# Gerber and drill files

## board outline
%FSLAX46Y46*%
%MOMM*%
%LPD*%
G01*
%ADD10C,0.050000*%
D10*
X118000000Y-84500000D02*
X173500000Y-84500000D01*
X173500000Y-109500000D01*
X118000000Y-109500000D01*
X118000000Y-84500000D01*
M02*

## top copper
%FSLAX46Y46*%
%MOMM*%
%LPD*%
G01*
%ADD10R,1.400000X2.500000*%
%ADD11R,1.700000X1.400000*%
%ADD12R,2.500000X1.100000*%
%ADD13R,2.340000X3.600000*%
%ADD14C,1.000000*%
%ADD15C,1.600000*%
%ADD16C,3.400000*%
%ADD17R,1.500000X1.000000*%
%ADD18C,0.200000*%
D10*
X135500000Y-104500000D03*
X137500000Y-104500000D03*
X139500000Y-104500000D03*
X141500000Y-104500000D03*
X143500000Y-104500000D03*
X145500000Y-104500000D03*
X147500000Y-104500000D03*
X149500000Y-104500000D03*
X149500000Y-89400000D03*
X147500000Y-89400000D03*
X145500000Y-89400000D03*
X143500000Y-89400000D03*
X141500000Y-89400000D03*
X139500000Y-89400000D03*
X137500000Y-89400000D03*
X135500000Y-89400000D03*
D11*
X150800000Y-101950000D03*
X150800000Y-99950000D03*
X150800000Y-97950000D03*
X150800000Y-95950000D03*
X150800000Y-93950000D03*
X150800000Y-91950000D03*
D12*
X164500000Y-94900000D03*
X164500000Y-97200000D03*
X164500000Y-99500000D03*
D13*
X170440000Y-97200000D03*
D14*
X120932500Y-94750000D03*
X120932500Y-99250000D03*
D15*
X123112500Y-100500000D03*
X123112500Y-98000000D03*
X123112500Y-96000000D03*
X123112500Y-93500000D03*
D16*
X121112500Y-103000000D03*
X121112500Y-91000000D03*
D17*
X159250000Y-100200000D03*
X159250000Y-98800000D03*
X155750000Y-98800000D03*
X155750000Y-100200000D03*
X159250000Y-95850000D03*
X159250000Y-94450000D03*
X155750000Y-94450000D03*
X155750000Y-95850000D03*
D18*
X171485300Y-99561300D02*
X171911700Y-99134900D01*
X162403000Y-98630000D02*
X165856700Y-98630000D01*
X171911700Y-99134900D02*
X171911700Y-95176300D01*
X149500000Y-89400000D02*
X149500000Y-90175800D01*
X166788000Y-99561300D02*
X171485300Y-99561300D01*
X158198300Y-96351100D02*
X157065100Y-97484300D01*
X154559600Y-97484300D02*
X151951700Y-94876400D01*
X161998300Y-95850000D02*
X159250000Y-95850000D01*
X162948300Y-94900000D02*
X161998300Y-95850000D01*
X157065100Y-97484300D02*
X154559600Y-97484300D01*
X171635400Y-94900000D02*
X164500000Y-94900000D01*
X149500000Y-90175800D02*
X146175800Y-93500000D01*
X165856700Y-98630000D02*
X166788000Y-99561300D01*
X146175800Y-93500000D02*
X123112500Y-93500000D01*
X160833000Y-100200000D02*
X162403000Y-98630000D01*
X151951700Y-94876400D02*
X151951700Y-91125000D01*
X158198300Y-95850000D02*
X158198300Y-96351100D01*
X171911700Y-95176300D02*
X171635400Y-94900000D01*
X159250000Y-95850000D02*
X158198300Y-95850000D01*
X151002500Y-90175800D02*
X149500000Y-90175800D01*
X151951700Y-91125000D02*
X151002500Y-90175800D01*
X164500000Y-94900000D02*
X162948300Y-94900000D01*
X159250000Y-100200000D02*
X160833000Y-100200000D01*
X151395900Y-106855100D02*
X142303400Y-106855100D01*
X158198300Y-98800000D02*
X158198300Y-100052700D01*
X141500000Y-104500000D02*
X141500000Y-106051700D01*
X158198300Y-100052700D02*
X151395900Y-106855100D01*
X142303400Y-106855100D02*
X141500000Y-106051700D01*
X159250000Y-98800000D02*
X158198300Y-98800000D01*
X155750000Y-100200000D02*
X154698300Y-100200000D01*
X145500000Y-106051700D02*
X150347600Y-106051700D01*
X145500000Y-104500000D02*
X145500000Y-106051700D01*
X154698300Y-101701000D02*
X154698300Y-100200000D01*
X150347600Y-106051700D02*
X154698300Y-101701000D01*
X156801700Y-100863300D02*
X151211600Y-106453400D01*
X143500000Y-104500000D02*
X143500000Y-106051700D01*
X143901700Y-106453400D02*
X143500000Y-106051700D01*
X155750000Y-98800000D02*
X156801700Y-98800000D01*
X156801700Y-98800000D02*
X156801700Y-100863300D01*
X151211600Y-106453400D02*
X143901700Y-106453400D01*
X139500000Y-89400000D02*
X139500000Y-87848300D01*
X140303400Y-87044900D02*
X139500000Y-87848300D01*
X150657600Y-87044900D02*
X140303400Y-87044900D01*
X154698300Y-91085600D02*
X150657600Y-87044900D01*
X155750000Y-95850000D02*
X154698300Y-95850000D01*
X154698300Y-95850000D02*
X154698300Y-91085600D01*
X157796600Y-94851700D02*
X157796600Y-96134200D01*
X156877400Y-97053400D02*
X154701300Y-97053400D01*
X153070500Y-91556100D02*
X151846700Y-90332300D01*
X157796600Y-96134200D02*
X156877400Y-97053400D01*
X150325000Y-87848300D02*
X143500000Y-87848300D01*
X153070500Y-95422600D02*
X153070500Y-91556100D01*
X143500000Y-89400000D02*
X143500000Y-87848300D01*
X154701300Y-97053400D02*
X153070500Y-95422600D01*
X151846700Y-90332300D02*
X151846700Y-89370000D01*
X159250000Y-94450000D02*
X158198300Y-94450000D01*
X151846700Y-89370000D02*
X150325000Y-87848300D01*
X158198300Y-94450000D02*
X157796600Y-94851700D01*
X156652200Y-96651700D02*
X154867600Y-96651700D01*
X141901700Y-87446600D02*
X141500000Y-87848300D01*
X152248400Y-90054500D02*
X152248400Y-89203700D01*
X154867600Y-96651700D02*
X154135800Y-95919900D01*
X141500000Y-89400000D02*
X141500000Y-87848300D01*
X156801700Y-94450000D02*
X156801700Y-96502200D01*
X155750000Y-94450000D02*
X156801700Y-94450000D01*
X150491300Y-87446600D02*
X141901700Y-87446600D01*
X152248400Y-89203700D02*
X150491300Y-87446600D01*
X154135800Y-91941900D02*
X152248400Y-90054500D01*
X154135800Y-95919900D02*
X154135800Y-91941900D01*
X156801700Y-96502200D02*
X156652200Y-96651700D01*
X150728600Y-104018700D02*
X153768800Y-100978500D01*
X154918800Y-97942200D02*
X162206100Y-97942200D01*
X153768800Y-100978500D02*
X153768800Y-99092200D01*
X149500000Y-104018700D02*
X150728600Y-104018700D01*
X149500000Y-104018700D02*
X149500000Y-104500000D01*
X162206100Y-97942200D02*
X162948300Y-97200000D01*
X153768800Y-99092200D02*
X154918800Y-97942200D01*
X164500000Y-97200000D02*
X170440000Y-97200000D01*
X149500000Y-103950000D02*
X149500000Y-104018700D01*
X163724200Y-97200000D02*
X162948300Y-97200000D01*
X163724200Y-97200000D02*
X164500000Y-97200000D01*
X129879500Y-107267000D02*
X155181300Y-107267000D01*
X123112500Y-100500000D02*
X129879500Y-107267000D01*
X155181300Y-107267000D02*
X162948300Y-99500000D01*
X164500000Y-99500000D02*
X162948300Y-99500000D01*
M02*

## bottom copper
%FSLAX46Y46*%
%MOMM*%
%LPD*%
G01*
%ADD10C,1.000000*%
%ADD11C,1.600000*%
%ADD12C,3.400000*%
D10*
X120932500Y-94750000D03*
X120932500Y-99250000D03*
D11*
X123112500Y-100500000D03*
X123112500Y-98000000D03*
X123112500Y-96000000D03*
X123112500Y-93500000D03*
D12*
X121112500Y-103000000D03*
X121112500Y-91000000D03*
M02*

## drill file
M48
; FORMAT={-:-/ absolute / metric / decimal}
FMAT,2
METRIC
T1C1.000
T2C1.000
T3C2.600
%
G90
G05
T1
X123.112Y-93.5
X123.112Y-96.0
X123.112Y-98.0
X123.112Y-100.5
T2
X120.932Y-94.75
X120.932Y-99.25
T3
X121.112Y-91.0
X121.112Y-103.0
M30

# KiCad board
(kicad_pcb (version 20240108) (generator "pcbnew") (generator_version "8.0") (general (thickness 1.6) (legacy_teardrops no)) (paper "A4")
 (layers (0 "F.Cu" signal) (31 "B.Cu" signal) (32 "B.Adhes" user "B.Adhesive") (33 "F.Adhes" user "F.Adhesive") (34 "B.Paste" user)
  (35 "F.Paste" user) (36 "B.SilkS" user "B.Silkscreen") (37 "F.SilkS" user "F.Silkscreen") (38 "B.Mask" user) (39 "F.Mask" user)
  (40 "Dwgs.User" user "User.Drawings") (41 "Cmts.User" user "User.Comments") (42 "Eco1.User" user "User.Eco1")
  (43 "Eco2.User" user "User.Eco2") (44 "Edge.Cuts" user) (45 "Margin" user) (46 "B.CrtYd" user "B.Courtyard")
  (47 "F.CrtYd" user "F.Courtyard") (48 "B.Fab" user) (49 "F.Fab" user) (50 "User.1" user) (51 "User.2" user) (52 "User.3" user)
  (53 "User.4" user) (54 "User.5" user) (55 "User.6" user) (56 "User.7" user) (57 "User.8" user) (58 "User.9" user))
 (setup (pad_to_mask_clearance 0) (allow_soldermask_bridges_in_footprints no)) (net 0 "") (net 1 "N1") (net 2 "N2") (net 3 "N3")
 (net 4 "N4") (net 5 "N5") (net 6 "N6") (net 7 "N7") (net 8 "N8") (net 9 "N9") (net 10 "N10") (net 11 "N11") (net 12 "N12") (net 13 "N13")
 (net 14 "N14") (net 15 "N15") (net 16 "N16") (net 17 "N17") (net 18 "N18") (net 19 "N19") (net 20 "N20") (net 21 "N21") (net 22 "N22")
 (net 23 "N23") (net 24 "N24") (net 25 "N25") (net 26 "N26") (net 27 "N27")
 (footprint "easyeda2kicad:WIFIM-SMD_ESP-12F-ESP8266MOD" (layer "F.Cu") (at 143.15 96.95)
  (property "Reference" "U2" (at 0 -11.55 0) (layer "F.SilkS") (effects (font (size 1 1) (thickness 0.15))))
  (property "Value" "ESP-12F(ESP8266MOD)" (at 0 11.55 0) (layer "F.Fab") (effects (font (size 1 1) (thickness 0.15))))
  (pad "1" smd rect (at -7.65 7.55 90) (size 2.5 1.4) (layers "F.Cu" "F.Paste" "F.Mask") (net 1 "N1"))
  (pad "2" smd rect (at -5.65 7.55 90) (size 2.5 1.4) (layers "F.Cu" "F.Paste" "F.Mask") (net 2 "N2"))
  (pad "3" smd rect (at -3.65 7.55 90) (size 2.5 1.4) (layers "F.Cu" "F.Paste" "F.Mask") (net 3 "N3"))
  (pad "4" smd rect (at -1.65 7.55 90) (size 2.5 1.4) (layers "F.Cu" "F.Paste" "F.Mask") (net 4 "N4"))
  (pad "5" smd rect (at 0.35 7.55 90) (size 2.5 1.4) (layers "F.Cu" "F.Paste" "F.Mask") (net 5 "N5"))
  (pad "6" smd rect (at 2.35 7.55 90) (size 2.5 1.4) (layers "F.Cu" "F.Paste" "F.Mask") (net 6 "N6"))
  (pad "7" smd rect (at 4.35 7.55 90) (size 2.5 1.4) (layers "F.Cu" "F.Paste" "F.Mask") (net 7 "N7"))
  (pad "8" smd rect (at 6.35 7.55 90) (size 2.5 1.4) (layers "F.Cu" "F.Paste" "F.Mask") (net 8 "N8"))
  (pad "9" smd rect (at 6.35 -7.55 270) (size 2.5 1.4) (layers "F.Cu" "F.Paste" "F.Mask") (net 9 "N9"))
  (pad "10" smd rect (at 4.35 -7.55 270) (size 2.5 1.4) (layers "F.Cu" "F.Paste" "F.Mask") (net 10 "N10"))
  (pad "11" smd rect (at 2.35 -7.55 270) (size 2.5 1.4) (layers "F.Cu" "F.Paste" "F.Mask") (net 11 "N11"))
  (pad "12" smd rect (at 0.35 -7.55 270) (size 2.5 1.4) (layers "F.Cu" "F.Paste" "F.Mask") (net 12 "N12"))
  (pad "13" smd rect (at -1.65 -7.55 270) (size 2.5 1.4) (layers "F.Cu" "F.Paste" "F.Mask") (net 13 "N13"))
  (pad "14" smd rect (at -3.65 -7.55 270) (size 2.5 1.4) (layers "F.Cu" "F.Paste" "F.Mask") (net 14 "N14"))
  (pad "15" smd rect (at -5.65 -7.55 270) (size 2.5 1.4) (layers "F.Cu" "F.Paste" "F.Mask") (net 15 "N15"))
  (pad "16" smd rect (at -7.65 -7.55 270) (size 2.5 1.4) (layers "F.Cu" "F.Paste" "F.Mask") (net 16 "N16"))
  (pad "17" smd rect (at 7.65 5 180) (size 1.7 1.4) (layers "F.Cu" "F.Paste" "F.Mask") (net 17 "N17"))
  (pad "18" smd rect (at 7.65 3 180) (size 1.7 1.4) (layers "F.Cu" "F.Paste" "F.Mask") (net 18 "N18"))
  (pad "19" smd rect (at 7.65 1 180) (size 1.7 1.4) (layers "F.Cu" "F.Paste" "F.Mask") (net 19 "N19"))
  (pad "20" smd rect (at 7.65 -1 180) (size 1.7 1.4) (layers "F.Cu" "F.Paste" "F.Mask") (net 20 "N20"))
  (pad "21" smd rect (at 7.65 -3 180) (size 1.7 1.4) (layers "F.Cu" "F.Paste" "F.Mask") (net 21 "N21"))
  (pad "22" smd rect (at 7.65 -5 180) (size 1.7 1.4) (layers "F.Cu" "F.Paste" "F.Mask") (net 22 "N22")))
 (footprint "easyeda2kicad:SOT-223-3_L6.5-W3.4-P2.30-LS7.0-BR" (layer "F.Cu") (at 167.47 97.2 180)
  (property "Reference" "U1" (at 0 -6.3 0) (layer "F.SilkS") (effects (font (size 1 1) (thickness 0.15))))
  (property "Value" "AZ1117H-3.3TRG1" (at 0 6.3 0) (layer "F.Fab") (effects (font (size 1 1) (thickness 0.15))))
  (pad "1" smd rect (at 2.97 2.3 180) (size 2.5 1.1) (layers "F.Cu" "F.Paste" "F.Mask") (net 9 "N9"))
  (pad "2" smd rect (at 2.97 0 180) (size 2.5 1.1) (layers "F.Cu" "F.Paste" "F.Mask") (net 8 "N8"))
  (pad "3" smd rect (at 2.97 -2.3 180) (size 2.5 1.1) (layers "F.Cu" "F.Paste" "F.Mask") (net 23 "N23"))
  (pad "4" smd rect (at -2.97 0 180) (size 2.34 3.6) (layers "F.Cu" "F.Paste" "F.Mask") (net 8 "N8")))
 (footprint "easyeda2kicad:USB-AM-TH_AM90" (layer "F.Cu") (at 122.1125 97 -90)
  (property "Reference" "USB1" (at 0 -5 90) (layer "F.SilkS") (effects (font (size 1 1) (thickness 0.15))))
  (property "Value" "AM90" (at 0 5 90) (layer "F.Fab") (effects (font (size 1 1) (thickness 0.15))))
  (pad "" thru_hole circle (at -2.25 1.18 270) (size 1 1) (drill 1) (layers "*.Cu" "*.Mask") (remove_unused_layers no))
  (pad "" thru_hole circle (at 2.25 1.18 270) (size 1 1) (drill 1) (layers "*.Cu" "*.Mask") (remove_unused_layers no))
  (pad "1" thru_hole circle (at 3.5 -1 180) (size 1.6 1.6) (drill 0.999998) (layers "*.Cu" "*.Mask") (remove_unused_layers no)
   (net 23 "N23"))
  (pad "2" thru_hole circle (at 1 -1 180) (size 1.6 1.6) (drill 0.999998) (layers "*.Cu" "*.Mask") (remove_unused_layers no) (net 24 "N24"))
  (pad "3" thru_hole circle (at -1 -1 180) (size 1.6 1.6) (drill 0.999998) (layers "*.Cu" "*.Mask") (remove_unused_layers no) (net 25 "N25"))
  (pad "4" thru_hole circle (at -3.5 -1 180) (size 1.6 1.6) (drill 0.999998) (layers "*.Cu" "*.Mask") (remove_unused_layers no) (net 9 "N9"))
  (pad "MH1" thru_hole circle (at 6 1 180) (size 3.4 3.4) (drill 2.599995) (layers "*.Cu" "*.Mask") (remove_unused_layers no) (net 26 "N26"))
  (pad "MH2" thru_hole circle (at -6 1 180) (size 3.4 3.4) (drill 2.599995) (layers "*.Cu" "*.Mask") (remove_unused_layers no)
   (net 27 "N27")))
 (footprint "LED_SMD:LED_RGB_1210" (layer "F.Cu") (at 157.5 99.5 180)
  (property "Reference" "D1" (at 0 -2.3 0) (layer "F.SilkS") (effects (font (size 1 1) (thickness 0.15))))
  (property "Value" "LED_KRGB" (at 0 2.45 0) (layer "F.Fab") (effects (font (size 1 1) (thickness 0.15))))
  (pad "1" smd rect (at -1.75 -0.7) (size 1.5 1) (layers "F.Cu" "F.Paste" "F.Mask") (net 9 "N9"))
  (pad "2" smd rect (at -1.75 0.7) (size 1.5 1) (layers "F.Cu" "F.Paste" "F.Mask") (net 4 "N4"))
  (pad "3" smd rect (at 1.75 0.7) (size 1.5 1) (layers "F.Cu" "F.Paste" "F.Mask") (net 5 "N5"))
  (pad "4" smd rect (at 1.75 -0.7) (size 1.5 1) (layers "F.Cu" "F.Paste" "F.Mask") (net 6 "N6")))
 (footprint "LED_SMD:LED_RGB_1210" (layer "F.Cu") (at 157.5 95.15 180)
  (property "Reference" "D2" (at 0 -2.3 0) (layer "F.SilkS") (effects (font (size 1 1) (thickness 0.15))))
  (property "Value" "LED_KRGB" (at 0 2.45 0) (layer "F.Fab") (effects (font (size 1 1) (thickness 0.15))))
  (pad "1" smd rect (at -1.75 -0.7) (size 1.5 1) (layers "F.Cu" "F.Paste" "F.Mask") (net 9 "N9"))
  (pad "2" smd rect (at -1.75 0.7) (size 1.5 1) (layers "F.Cu" "F.Paste" "F.Mask") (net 12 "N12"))
  (pad "3" smd rect (at 1.75 0.7) (size 1.5 1) (layers "F.Cu" "F.Paste" "F.Mask") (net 13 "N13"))
  (pad "4" smd rect (at 1.75 -0.7) (size 1.5 1) (layers "F.Cu" "F.Paste" "F.Mask") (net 14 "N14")))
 (gr_rect (start 118 84.5) (end 173.5 109.5) (stroke (width 0.05) (type default)) (fill none) (layer "Edge.Cuts"))
 (segment (start 171.4853 99.5613) (end 171.9117 99.1349) (width 0.2) (layer "F.Cu") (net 9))
 (segment (start 162.403 98.63) (end 165.8567 98.63) (width 0.2) (layer "F.Cu") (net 9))
 (segment (start 171.9117 99.1349) (end 171.9117 95.1763) (width 0.2) (layer "F.Cu") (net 9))
 (segment (start 149.5 89.4) (end 149.5 90.1758) (width 0.2) (layer "F.Cu") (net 9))
 (segment (start 166.788 99.5613) (end 171.4853 99.5613) (width 0.2) (layer "F.Cu") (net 9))
 (segment (start 158.1983 96.3511) (end 157.0651 97.4843) (width 0.2) (layer "F.Cu") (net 9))
 (segment (start 154.5596 97.4843) (end 151.9517 94.8764) (width 0.2) (layer "F.Cu") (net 9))
 (segment (start 161.9983 95.85) (end 159.25 95.85) (width 0.2) (layer "F.Cu") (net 9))
 (segment (start 162.9483 94.9) (end 161.9983 95.85) (width 0.2) (layer "F.Cu") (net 9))
 (segment (start 157.0651 97.4843) (end 154.5596 97.4843) (width 0.2) (layer "F.Cu") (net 9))
 (segment (start 171.6354 94.9) (end 164.5 94.9) (width 0.2) (layer "F.Cu") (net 9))
 (segment (start 149.5 90.1758) (end 146.1758 93.5) (width 0.2) (layer "F.Cu") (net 9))
 (segment (start 165.8567 98.63) (end 166.788 99.5613) (width 0.2) (layer "F.Cu") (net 9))
 (segment (start 146.1758 93.5) (end 123.1125 93.5) (width 0.2) (layer "F.Cu") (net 9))
 (segment (start 160.833 100.2) (end 162.403 98.63) (width 0.2) (layer "F.Cu") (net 9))
 (segment (start 151.9517 94.8764) (end 151.9517 91.125) (width 0.2) (layer "F.Cu") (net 9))
 (segment (start 158.1983 95.85) (end 158.1983 96.3511) (width 0.2) (layer "F.Cu") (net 9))
 (segment (start 171.9117 95.1763) (end 171.6354 94.9) (width 0.2) (layer "F.Cu") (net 9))
 (segment (start 159.25 95.85) (end 158.1983 95.85) (width 0.2) (layer "F.Cu") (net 9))
 (segment (start 151.0025 90.1758) (end 149.5 90.1758) (width 0.2) (layer "F.Cu") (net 9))
 (segment (start 151.9517 91.125) (end 151.0025 90.1758) (width 0.2) (layer "F.Cu") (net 9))
 (segment (start 164.5 94.9) (end 162.9483 94.9) (width 0.2) (layer "F.Cu") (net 9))
 (segment (start 159.25 100.2) (end 160.833 100.2) (width 0.2) (layer "F.Cu") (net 9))
 (segment (start 151.3959 106.8551) (end 142.3034 106.8551) (width 0.2) (layer "F.Cu") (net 4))
 (segment (start 158.1983 98.8) (end 158.1983 100.0527) (width 0.2) (layer "F.Cu") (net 4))
 (segment (start 141.5 104.5) (end 141.5 106.0517) (width 0.2) (layer "F.Cu") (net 4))
 (segment (start 158.1983 100.0527) (end 151.3959 106.8551) (width 0.2) (layer "F.Cu") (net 4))
 (segment (start 142.3034 106.8551) (end 141.5 106.0517) (width 0.2) (layer "F.Cu") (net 4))
 (segment (start 159.25 98.8) (end 158.1983 98.8) (width 0.2) (layer "F.Cu") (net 4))
 (segment (start 155.75 100.2) (end 154.6983 100.2) (width 0.2) (layer "F.Cu") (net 6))
 (segment (start 145.5 106.0517) (end 150.3476 106.0517) (width 0.2) (layer "F.Cu") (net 6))
 (segment (start 145.5 104.5) (end 145.5 106.0517) (width 0.2) (layer "F.Cu") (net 6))
 (segment (start 154.6983 101.701) (end 154.6983 100.2) (width 0.2) (layer "F.Cu") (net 6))
 (segment (start 150.3476 106.0517) (end 154.6983 101.701) (width 0.2) (layer "F.Cu") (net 6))
 (segment (start 156.8017 100.8633) (end 151.2116 106.4534) (width 0.2) (layer "F.Cu") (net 5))
 (segment (start 143.5 104.5) (end 143.5 106.0517) (width 0.2) (layer "F.Cu") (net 5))
 (segment (start 143.9017 106.4534) (end 143.5 106.0517) (width 0.2) (layer "F.Cu") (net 5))
 (segment (start 155.75 98.8) (end 156.8017 98.8) (width 0.2) (layer "F.Cu") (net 5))
 (segment (start 156.8017 98.8) (end 156.8017 100.8633) (width 0.2) (layer "F.Cu") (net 5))
 (segment (start 151.2116 106.4534) (end 143.9017 106.4534) (width 0.2) (layer "F.Cu") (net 5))
 (segment (start 139.5 89.4) (end 139.5 87.8483) (width 0.2) (layer "F.Cu") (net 14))
 (segment (start 140.3034 87.0449) (end 139.5 87.8483) (width 0.2) (layer "F.Cu") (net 14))
 (segment (start 150.6576 87.0449) (end 140.3034 87.0449) (width 0.2) (layer "F.Cu") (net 14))
 (segment (start 154.6983 91.0856) (end 150.6576 87.0449) (width 0.2) (layer "F.Cu") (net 14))
 (segment (start 155.75 95.85) (end 154.6983 95.85) (width 0.2) (layer "F.Cu") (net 14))
 (segment (start 154.6983 95.85) (end 154.6983 91.0856) (width 0.2) (layer "F.Cu") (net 14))
 (segment (start 157.7966 94.8517) (end 157.7966 96.1342) (width 0.2) (layer "F.Cu") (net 12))
 (segment (start 156.8774 97.0534) (end 154.7013 97.0534) (width 0.2) (layer "F.Cu") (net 12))
 (segment (start 153.0705 91.5561) (end 151.8467 90.3323) (width 0.2) (layer "F.Cu") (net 12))
 (segment (start 157.7966 96.1342) (end 156.8774 97.0534) (width 0.2) (layer "F.Cu") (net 12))
 (segment (start 150.325 87.8483) (end 143.5 87.8483) (width 0.2) (layer "F.Cu") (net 12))
 (segment (start 153.0705 95.4226) (end 153.0705 91.5561) (width 0.2) (layer "F.Cu") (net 12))
 (segment (start 143.5 89.4) (end 143.5 87.8483) (width 0.2) (layer "F.Cu") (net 12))
 (segment (start 154.7013 97.0534) (end 153.0705 95.4226) (width 0.2) (layer "F.Cu") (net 12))
 (segment (start 151.8467 90.3323) (end 151.8467 89.37) (width 0.2) (layer "F.Cu") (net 12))
 (segment (start 159.25 94.45) (end 158.1983 94.45) (width 0.2) (layer "F.Cu") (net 12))
 (segment (start 151.8467 89.37) (end 150.325 87.8483) (width 0.2) (layer "F.Cu") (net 12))
 (segment (start 158.1983 94.45) (end 157.7966 94.8517) (width 0.2) (layer "F.Cu") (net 12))
 (segment (start 156.6522 96.6517) (end 154.8676 96.6517) (width 0.2) (layer "F.Cu") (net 13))
 (segment (start 141.9017 87.4466) (end 141.5 87.8483) (width 0.2) (layer "F.Cu") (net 13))
 (segment (start 152.2484 90.0545) (end 152.2484 89.2037) (width 0.2) (layer "F.Cu") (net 13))
 (segment (start 154.8676 96.6517) (end 154.1358 95.9199) (width 0.2) (layer "F.Cu") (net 13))
 (segment (start 141.5 89.4) (end 141.5 87.8483) (width 0.2) (layer "F.Cu") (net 13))
 (segment (start 156.8017 94.45) (end 156.8017 96.5022) (width 0.2) (layer "F.Cu") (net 13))
 (segment (start 155.75 94.45) (end 156.8017 94.45) (width 0.2) (layer "F.Cu") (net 13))
 (segment (start 150.4913 87.4466) (end 141.9017 87.4466) (width 0.2) (layer "F.Cu") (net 13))
 (segment (start 152.2484 89.2037) (end 150.4913 87.4466) (width 0.2) (layer "F.Cu") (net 13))
 (segment (start 154.1358 91.9419) (end 152.2484 90.0545) (width 0.2) (layer "F.Cu") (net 13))
 (segment (start 154.1358 95.9199) (end 154.1358 91.9419) (width 0.2) (layer "F.Cu") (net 13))
 (segment (start 156.8017 96.5022) (end 156.6522 96.6517) (width 0.2) (layer "F.Cu") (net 13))
 (segment (start 150.7286 104.0187) (end 153.7688 100.9785) (width 0.2) (layer "F.Cu") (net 8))
 (segment (start 154.9188 97.9422) (end 162.2061 97.9422) (width 0.2) (layer "F.Cu") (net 8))
 (segment (start 153.7688 100.9785) (end 153.7688 99.0922) (width 0.2) (layer "F.Cu") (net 8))
 (segment (start 149.5 104.0187) (end 150.7286 104.0187) (width 0.2) (layer "F.Cu") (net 8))
 (segment (start 149.5 104.0187) (end 149.5 104.5) (width 0.2) (layer "F.Cu") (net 8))
 (segment (start 162.2061 97.9422) (end 162.9483 97.2) (width 0.2) (layer "F.Cu") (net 8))
 (segment (start 153.7688 99.0922) (end 154.9188 97.9422) (width 0.2) (layer "F.Cu") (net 8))
 (segment (start 164.5 97.2) (end 170.44 97.2) (width 0.2) (layer "F.Cu") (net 8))
 (segment (start 149.5 103.95) (end 149.5 104.0187) (width 0.2) (layer "F.Cu") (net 8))
 (segment (start 163.7242 97.2) (end 162.9483 97.2) (width 0.2) (layer "F.Cu") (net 8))
 (segment (start 163.7242 97.2) (end 164.5 97.2) (width 0.2) (layer "F.Cu") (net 8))
 (segment (start 129.8795 107.267) (end 155.1813 107.267) (width 0.2) (layer "F.Cu") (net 23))
 (segment (start 123.1125 100.5) (end 129.8795 107.267) (width 0.2) (layer "F.Cu") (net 23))
 (segment (start 155.1813 107.267) (end 162.9483 99.5) (width 0.2) (layer "F.Cu") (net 23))
 (segment (start 164.5 99.5) (end 162.9483 99.5) (width 0.2) (layer "F.Cu") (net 23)))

